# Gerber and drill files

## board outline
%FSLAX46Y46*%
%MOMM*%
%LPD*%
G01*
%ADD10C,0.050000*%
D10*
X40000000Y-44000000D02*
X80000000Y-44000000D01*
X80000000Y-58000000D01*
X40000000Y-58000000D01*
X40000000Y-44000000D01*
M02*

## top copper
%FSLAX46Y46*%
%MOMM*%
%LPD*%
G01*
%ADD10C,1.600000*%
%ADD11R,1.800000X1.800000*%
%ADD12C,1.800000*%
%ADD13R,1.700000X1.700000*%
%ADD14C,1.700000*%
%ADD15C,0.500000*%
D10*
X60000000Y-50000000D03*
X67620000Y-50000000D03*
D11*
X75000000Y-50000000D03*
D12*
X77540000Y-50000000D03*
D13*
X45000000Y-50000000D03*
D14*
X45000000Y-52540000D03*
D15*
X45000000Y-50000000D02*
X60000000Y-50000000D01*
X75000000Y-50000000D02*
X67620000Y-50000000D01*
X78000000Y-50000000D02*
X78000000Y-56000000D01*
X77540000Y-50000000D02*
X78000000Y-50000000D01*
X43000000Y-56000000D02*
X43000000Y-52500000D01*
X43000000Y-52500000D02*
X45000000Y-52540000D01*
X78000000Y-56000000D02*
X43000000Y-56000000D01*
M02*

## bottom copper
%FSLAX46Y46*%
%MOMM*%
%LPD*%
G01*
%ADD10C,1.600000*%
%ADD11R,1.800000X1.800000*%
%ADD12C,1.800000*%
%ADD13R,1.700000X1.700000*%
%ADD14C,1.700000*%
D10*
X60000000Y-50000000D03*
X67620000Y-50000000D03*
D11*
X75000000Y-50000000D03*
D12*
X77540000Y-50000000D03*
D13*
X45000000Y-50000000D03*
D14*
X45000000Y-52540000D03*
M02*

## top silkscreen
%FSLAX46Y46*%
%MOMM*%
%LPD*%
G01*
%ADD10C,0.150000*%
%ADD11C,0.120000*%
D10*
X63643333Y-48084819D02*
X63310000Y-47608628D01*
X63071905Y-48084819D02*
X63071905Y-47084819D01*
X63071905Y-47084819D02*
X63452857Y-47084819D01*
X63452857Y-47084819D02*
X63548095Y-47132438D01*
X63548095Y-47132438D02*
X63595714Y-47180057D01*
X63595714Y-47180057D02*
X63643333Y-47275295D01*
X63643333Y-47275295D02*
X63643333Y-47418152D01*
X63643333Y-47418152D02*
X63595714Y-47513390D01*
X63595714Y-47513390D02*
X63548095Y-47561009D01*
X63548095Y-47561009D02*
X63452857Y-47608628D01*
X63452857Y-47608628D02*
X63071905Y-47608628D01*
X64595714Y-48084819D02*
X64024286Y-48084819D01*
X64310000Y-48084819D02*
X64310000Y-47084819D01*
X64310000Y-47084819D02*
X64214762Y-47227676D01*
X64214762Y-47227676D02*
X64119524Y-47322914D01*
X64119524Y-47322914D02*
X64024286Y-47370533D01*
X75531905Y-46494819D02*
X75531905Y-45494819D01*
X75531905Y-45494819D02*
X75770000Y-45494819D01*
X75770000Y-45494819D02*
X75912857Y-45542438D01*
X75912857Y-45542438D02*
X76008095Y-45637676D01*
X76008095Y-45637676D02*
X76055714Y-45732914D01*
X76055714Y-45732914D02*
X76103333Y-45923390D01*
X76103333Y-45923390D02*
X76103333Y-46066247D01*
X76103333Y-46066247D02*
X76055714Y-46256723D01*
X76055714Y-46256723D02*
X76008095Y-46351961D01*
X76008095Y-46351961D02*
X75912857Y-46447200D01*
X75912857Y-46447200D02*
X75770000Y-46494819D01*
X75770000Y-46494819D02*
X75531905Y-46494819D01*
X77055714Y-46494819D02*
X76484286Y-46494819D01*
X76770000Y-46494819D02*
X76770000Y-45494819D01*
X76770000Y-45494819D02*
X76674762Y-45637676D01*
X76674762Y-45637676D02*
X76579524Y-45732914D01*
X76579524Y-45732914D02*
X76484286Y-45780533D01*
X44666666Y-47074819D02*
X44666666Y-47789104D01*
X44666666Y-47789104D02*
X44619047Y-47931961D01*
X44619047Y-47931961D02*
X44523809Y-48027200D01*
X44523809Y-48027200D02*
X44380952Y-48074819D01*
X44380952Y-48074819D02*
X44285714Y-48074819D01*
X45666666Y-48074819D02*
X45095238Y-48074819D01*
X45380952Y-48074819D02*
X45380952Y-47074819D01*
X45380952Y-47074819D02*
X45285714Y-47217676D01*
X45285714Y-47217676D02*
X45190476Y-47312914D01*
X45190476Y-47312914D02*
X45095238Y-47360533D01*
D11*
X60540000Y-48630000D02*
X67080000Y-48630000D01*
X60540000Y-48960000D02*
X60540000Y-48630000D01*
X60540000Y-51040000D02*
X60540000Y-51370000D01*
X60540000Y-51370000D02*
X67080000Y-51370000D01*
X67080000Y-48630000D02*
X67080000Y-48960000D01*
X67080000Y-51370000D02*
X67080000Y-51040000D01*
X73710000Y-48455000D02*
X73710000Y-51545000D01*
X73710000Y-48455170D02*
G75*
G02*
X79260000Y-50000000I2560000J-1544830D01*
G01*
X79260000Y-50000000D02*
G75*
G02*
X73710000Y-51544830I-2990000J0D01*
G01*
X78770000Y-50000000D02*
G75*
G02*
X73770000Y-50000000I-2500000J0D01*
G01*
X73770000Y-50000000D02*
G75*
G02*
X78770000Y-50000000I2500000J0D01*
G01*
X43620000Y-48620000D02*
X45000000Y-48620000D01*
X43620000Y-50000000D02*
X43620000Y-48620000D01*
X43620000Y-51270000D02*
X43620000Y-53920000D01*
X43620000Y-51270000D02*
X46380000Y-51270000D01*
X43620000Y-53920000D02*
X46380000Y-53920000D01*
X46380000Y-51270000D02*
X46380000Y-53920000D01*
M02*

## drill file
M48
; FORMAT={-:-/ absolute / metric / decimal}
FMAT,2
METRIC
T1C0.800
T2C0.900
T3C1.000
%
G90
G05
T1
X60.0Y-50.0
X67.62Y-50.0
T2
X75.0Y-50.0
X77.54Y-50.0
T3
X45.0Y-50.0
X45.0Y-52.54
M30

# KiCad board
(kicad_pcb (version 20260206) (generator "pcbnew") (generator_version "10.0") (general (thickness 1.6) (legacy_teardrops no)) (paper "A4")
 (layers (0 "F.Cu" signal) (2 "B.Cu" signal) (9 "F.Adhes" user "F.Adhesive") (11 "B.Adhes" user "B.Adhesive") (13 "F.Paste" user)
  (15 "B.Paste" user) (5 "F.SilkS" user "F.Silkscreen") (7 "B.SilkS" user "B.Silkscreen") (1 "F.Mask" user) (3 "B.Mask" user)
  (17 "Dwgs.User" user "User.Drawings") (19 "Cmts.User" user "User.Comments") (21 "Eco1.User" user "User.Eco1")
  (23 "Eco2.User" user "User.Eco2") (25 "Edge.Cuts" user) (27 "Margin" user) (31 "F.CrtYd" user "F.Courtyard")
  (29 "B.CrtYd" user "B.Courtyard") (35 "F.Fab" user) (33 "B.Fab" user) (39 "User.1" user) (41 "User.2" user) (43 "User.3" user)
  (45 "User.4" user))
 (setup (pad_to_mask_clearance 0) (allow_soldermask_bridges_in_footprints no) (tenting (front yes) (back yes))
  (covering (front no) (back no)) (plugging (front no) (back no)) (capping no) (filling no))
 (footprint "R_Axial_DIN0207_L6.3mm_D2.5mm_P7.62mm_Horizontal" (layer "F.Cu") (at 60 50)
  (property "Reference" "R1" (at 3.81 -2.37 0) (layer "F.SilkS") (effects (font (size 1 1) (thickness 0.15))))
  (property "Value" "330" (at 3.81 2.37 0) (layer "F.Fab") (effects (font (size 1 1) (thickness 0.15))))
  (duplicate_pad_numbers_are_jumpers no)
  (fp_line (start 0.54 -1.37) (end 7.08 -1.37) (stroke (width 0.12) (type solid)) (layer "F.SilkS"))
  (fp_line (start 0.54 -1.04) (end 0.54 -1.37) (stroke (width 0.12) (type solid)) (layer "F.SilkS"))
  (fp_line (start 0.54 1.04) (end 0.54 1.37) (stroke (width 0.12) (type solid)) (layer "F.SilkS"))
  (fp_line (start 0.54 1.37) (end 7.08 1.37) (stroke (width 0.12) (type solid)) (layer "F.SilkS"))
  (fp_line (start 7.08 -1.37) (end 7.08 -1.04) (stroke (width 0.12) (type solid)) (layer "F.SilkS"))
  (fp_line (start 7.08 1.37) (end 7.08 1.04) (stroke (width 0.12) (type solid)) (layer "F.SilkS"))
  (pad "1" thru_hole circle (at 0 0) (size 1.6 1.6) (drill 0.8) (layers "*.Cu" "*.Mask") (remove_unused_layers no) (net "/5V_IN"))
  (pad "2" thru_hole circle (at 7.62 0) (size 1.6 1.6) (drill 0.8) (layers "*.Cu" "*.Mask") (remove_unused_layers no) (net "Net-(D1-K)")))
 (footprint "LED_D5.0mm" (layer "F.Cu") (at 75 50)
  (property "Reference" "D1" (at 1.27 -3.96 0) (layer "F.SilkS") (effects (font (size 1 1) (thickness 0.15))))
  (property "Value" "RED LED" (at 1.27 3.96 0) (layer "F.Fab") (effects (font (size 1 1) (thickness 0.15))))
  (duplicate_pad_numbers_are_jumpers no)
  (fp_line (start -1.29 -1.545) (end -1.29 1.545) (stroke (width 0.12) (type solid)) (layer "F.SilkS"))
  (fp_arc (start -1.29 -1.54483) (mid 2.071779 -2.880495) (end 4.26 0) (stroke (width 0.12) (type solid)) (layer "F.SilkS"))
  (fp_arc (start 4.26 0) (mid 2.071779 2.880495) (end -1.29 1.54483) (stroke (width 0.12) (type solid)) (layer "F.SilkS"))
  (fp_circle (center 1.27 0) (end 3.77 0) (stroke (width 0.12) (type solid)) (fill no) (layer "F.SilkS"))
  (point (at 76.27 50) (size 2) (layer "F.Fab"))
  (pad "1" thru_hole rect (at 0 0) (size 1.8 1.8) (drill 0.9) (layers "*.Cu" "*.Mask") (remove_unused_layers no) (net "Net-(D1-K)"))
  (pad "2" thru_hole circle (at 2.54 0) (size 1.8 1.8) (drill 0.9) (layers "*.Cu" "*.Mask") (remove_unused_layers no) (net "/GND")))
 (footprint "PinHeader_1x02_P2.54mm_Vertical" (layer "F.Cu") (at 45 50)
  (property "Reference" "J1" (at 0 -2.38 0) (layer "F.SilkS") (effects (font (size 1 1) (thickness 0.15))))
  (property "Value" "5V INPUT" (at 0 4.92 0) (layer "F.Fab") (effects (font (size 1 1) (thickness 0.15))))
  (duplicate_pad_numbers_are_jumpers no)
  (fp_line (start -1.38 -1.38) (end 0 -1.38) (stroke (width 0.12) (type solid)) (layer "F.SilkS"))
  (fp_line (start -1.38 0) (end -1.38 -1.38) (stroke (width 0.12) (type solid)) (layer "F.SilkS"))
  (fp_line (start -1.38 1.27) (end -1.38 3.92) (stroke (width 0.12) (type solid)) (layer "F.SilkS"))
  (fp_line (start -1.38 1.27) (end 1.38 1.27) (stroke (width 0.12) (type solid)) (layer "F.SilkS"))
  (fp_line (start -1.38 3.92) (end 1.38 3.92) (stroke (width 0.12) (type solid)) (layer "F.SilkS"))
  (fp_line (start 1.38 1.27) (end 1.38 3.92) (stroke (width 0.12) (type solid)) (layer "F.SilkS"))
  (pad "1" thru_hole rect (at 0 0) (size 1.7 1.7) (drill 1) (layers "*.Cu" "*.Mask") (remove_unused_layers no) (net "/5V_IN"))
  (pad "2" thru_hole circle (at 0 2.54) (size 1.7 1.7) (drill 1) (layers "*.Cu" "*.Mask") (remove_unused_layers no) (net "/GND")))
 (gr_rect (start 40 44) (end 80 58) (stroke (width 0.05) (type default)) (fill no) (layer "Edge.Cuts"))
 (segment (start 45 50) (end 60 50) (width 0.5) (layer "F.Cu") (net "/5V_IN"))
 (segment (start 75 50) (end 67.62 50) (width 0.5) (layer "F.Cu") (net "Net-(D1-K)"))
 (segment (start 78 50) (end 78 56) (width 0.5) (layer "F.Cu") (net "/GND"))
 (segment (start 77.54 50) (end 78 50) (width 0.5) (layer "F.Cu") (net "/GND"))
 (segment (start 43 56) (end 43 52.5) (width 0.5) (layer "F.Cu") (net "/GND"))
 (segment (start 43 52.5) (end 45 52.54) (width 0.5) (layer "F.Cu") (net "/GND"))
 (segment (start 78 56) (end 43 56) (width 0.5) (layer "F.Cu") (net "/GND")))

